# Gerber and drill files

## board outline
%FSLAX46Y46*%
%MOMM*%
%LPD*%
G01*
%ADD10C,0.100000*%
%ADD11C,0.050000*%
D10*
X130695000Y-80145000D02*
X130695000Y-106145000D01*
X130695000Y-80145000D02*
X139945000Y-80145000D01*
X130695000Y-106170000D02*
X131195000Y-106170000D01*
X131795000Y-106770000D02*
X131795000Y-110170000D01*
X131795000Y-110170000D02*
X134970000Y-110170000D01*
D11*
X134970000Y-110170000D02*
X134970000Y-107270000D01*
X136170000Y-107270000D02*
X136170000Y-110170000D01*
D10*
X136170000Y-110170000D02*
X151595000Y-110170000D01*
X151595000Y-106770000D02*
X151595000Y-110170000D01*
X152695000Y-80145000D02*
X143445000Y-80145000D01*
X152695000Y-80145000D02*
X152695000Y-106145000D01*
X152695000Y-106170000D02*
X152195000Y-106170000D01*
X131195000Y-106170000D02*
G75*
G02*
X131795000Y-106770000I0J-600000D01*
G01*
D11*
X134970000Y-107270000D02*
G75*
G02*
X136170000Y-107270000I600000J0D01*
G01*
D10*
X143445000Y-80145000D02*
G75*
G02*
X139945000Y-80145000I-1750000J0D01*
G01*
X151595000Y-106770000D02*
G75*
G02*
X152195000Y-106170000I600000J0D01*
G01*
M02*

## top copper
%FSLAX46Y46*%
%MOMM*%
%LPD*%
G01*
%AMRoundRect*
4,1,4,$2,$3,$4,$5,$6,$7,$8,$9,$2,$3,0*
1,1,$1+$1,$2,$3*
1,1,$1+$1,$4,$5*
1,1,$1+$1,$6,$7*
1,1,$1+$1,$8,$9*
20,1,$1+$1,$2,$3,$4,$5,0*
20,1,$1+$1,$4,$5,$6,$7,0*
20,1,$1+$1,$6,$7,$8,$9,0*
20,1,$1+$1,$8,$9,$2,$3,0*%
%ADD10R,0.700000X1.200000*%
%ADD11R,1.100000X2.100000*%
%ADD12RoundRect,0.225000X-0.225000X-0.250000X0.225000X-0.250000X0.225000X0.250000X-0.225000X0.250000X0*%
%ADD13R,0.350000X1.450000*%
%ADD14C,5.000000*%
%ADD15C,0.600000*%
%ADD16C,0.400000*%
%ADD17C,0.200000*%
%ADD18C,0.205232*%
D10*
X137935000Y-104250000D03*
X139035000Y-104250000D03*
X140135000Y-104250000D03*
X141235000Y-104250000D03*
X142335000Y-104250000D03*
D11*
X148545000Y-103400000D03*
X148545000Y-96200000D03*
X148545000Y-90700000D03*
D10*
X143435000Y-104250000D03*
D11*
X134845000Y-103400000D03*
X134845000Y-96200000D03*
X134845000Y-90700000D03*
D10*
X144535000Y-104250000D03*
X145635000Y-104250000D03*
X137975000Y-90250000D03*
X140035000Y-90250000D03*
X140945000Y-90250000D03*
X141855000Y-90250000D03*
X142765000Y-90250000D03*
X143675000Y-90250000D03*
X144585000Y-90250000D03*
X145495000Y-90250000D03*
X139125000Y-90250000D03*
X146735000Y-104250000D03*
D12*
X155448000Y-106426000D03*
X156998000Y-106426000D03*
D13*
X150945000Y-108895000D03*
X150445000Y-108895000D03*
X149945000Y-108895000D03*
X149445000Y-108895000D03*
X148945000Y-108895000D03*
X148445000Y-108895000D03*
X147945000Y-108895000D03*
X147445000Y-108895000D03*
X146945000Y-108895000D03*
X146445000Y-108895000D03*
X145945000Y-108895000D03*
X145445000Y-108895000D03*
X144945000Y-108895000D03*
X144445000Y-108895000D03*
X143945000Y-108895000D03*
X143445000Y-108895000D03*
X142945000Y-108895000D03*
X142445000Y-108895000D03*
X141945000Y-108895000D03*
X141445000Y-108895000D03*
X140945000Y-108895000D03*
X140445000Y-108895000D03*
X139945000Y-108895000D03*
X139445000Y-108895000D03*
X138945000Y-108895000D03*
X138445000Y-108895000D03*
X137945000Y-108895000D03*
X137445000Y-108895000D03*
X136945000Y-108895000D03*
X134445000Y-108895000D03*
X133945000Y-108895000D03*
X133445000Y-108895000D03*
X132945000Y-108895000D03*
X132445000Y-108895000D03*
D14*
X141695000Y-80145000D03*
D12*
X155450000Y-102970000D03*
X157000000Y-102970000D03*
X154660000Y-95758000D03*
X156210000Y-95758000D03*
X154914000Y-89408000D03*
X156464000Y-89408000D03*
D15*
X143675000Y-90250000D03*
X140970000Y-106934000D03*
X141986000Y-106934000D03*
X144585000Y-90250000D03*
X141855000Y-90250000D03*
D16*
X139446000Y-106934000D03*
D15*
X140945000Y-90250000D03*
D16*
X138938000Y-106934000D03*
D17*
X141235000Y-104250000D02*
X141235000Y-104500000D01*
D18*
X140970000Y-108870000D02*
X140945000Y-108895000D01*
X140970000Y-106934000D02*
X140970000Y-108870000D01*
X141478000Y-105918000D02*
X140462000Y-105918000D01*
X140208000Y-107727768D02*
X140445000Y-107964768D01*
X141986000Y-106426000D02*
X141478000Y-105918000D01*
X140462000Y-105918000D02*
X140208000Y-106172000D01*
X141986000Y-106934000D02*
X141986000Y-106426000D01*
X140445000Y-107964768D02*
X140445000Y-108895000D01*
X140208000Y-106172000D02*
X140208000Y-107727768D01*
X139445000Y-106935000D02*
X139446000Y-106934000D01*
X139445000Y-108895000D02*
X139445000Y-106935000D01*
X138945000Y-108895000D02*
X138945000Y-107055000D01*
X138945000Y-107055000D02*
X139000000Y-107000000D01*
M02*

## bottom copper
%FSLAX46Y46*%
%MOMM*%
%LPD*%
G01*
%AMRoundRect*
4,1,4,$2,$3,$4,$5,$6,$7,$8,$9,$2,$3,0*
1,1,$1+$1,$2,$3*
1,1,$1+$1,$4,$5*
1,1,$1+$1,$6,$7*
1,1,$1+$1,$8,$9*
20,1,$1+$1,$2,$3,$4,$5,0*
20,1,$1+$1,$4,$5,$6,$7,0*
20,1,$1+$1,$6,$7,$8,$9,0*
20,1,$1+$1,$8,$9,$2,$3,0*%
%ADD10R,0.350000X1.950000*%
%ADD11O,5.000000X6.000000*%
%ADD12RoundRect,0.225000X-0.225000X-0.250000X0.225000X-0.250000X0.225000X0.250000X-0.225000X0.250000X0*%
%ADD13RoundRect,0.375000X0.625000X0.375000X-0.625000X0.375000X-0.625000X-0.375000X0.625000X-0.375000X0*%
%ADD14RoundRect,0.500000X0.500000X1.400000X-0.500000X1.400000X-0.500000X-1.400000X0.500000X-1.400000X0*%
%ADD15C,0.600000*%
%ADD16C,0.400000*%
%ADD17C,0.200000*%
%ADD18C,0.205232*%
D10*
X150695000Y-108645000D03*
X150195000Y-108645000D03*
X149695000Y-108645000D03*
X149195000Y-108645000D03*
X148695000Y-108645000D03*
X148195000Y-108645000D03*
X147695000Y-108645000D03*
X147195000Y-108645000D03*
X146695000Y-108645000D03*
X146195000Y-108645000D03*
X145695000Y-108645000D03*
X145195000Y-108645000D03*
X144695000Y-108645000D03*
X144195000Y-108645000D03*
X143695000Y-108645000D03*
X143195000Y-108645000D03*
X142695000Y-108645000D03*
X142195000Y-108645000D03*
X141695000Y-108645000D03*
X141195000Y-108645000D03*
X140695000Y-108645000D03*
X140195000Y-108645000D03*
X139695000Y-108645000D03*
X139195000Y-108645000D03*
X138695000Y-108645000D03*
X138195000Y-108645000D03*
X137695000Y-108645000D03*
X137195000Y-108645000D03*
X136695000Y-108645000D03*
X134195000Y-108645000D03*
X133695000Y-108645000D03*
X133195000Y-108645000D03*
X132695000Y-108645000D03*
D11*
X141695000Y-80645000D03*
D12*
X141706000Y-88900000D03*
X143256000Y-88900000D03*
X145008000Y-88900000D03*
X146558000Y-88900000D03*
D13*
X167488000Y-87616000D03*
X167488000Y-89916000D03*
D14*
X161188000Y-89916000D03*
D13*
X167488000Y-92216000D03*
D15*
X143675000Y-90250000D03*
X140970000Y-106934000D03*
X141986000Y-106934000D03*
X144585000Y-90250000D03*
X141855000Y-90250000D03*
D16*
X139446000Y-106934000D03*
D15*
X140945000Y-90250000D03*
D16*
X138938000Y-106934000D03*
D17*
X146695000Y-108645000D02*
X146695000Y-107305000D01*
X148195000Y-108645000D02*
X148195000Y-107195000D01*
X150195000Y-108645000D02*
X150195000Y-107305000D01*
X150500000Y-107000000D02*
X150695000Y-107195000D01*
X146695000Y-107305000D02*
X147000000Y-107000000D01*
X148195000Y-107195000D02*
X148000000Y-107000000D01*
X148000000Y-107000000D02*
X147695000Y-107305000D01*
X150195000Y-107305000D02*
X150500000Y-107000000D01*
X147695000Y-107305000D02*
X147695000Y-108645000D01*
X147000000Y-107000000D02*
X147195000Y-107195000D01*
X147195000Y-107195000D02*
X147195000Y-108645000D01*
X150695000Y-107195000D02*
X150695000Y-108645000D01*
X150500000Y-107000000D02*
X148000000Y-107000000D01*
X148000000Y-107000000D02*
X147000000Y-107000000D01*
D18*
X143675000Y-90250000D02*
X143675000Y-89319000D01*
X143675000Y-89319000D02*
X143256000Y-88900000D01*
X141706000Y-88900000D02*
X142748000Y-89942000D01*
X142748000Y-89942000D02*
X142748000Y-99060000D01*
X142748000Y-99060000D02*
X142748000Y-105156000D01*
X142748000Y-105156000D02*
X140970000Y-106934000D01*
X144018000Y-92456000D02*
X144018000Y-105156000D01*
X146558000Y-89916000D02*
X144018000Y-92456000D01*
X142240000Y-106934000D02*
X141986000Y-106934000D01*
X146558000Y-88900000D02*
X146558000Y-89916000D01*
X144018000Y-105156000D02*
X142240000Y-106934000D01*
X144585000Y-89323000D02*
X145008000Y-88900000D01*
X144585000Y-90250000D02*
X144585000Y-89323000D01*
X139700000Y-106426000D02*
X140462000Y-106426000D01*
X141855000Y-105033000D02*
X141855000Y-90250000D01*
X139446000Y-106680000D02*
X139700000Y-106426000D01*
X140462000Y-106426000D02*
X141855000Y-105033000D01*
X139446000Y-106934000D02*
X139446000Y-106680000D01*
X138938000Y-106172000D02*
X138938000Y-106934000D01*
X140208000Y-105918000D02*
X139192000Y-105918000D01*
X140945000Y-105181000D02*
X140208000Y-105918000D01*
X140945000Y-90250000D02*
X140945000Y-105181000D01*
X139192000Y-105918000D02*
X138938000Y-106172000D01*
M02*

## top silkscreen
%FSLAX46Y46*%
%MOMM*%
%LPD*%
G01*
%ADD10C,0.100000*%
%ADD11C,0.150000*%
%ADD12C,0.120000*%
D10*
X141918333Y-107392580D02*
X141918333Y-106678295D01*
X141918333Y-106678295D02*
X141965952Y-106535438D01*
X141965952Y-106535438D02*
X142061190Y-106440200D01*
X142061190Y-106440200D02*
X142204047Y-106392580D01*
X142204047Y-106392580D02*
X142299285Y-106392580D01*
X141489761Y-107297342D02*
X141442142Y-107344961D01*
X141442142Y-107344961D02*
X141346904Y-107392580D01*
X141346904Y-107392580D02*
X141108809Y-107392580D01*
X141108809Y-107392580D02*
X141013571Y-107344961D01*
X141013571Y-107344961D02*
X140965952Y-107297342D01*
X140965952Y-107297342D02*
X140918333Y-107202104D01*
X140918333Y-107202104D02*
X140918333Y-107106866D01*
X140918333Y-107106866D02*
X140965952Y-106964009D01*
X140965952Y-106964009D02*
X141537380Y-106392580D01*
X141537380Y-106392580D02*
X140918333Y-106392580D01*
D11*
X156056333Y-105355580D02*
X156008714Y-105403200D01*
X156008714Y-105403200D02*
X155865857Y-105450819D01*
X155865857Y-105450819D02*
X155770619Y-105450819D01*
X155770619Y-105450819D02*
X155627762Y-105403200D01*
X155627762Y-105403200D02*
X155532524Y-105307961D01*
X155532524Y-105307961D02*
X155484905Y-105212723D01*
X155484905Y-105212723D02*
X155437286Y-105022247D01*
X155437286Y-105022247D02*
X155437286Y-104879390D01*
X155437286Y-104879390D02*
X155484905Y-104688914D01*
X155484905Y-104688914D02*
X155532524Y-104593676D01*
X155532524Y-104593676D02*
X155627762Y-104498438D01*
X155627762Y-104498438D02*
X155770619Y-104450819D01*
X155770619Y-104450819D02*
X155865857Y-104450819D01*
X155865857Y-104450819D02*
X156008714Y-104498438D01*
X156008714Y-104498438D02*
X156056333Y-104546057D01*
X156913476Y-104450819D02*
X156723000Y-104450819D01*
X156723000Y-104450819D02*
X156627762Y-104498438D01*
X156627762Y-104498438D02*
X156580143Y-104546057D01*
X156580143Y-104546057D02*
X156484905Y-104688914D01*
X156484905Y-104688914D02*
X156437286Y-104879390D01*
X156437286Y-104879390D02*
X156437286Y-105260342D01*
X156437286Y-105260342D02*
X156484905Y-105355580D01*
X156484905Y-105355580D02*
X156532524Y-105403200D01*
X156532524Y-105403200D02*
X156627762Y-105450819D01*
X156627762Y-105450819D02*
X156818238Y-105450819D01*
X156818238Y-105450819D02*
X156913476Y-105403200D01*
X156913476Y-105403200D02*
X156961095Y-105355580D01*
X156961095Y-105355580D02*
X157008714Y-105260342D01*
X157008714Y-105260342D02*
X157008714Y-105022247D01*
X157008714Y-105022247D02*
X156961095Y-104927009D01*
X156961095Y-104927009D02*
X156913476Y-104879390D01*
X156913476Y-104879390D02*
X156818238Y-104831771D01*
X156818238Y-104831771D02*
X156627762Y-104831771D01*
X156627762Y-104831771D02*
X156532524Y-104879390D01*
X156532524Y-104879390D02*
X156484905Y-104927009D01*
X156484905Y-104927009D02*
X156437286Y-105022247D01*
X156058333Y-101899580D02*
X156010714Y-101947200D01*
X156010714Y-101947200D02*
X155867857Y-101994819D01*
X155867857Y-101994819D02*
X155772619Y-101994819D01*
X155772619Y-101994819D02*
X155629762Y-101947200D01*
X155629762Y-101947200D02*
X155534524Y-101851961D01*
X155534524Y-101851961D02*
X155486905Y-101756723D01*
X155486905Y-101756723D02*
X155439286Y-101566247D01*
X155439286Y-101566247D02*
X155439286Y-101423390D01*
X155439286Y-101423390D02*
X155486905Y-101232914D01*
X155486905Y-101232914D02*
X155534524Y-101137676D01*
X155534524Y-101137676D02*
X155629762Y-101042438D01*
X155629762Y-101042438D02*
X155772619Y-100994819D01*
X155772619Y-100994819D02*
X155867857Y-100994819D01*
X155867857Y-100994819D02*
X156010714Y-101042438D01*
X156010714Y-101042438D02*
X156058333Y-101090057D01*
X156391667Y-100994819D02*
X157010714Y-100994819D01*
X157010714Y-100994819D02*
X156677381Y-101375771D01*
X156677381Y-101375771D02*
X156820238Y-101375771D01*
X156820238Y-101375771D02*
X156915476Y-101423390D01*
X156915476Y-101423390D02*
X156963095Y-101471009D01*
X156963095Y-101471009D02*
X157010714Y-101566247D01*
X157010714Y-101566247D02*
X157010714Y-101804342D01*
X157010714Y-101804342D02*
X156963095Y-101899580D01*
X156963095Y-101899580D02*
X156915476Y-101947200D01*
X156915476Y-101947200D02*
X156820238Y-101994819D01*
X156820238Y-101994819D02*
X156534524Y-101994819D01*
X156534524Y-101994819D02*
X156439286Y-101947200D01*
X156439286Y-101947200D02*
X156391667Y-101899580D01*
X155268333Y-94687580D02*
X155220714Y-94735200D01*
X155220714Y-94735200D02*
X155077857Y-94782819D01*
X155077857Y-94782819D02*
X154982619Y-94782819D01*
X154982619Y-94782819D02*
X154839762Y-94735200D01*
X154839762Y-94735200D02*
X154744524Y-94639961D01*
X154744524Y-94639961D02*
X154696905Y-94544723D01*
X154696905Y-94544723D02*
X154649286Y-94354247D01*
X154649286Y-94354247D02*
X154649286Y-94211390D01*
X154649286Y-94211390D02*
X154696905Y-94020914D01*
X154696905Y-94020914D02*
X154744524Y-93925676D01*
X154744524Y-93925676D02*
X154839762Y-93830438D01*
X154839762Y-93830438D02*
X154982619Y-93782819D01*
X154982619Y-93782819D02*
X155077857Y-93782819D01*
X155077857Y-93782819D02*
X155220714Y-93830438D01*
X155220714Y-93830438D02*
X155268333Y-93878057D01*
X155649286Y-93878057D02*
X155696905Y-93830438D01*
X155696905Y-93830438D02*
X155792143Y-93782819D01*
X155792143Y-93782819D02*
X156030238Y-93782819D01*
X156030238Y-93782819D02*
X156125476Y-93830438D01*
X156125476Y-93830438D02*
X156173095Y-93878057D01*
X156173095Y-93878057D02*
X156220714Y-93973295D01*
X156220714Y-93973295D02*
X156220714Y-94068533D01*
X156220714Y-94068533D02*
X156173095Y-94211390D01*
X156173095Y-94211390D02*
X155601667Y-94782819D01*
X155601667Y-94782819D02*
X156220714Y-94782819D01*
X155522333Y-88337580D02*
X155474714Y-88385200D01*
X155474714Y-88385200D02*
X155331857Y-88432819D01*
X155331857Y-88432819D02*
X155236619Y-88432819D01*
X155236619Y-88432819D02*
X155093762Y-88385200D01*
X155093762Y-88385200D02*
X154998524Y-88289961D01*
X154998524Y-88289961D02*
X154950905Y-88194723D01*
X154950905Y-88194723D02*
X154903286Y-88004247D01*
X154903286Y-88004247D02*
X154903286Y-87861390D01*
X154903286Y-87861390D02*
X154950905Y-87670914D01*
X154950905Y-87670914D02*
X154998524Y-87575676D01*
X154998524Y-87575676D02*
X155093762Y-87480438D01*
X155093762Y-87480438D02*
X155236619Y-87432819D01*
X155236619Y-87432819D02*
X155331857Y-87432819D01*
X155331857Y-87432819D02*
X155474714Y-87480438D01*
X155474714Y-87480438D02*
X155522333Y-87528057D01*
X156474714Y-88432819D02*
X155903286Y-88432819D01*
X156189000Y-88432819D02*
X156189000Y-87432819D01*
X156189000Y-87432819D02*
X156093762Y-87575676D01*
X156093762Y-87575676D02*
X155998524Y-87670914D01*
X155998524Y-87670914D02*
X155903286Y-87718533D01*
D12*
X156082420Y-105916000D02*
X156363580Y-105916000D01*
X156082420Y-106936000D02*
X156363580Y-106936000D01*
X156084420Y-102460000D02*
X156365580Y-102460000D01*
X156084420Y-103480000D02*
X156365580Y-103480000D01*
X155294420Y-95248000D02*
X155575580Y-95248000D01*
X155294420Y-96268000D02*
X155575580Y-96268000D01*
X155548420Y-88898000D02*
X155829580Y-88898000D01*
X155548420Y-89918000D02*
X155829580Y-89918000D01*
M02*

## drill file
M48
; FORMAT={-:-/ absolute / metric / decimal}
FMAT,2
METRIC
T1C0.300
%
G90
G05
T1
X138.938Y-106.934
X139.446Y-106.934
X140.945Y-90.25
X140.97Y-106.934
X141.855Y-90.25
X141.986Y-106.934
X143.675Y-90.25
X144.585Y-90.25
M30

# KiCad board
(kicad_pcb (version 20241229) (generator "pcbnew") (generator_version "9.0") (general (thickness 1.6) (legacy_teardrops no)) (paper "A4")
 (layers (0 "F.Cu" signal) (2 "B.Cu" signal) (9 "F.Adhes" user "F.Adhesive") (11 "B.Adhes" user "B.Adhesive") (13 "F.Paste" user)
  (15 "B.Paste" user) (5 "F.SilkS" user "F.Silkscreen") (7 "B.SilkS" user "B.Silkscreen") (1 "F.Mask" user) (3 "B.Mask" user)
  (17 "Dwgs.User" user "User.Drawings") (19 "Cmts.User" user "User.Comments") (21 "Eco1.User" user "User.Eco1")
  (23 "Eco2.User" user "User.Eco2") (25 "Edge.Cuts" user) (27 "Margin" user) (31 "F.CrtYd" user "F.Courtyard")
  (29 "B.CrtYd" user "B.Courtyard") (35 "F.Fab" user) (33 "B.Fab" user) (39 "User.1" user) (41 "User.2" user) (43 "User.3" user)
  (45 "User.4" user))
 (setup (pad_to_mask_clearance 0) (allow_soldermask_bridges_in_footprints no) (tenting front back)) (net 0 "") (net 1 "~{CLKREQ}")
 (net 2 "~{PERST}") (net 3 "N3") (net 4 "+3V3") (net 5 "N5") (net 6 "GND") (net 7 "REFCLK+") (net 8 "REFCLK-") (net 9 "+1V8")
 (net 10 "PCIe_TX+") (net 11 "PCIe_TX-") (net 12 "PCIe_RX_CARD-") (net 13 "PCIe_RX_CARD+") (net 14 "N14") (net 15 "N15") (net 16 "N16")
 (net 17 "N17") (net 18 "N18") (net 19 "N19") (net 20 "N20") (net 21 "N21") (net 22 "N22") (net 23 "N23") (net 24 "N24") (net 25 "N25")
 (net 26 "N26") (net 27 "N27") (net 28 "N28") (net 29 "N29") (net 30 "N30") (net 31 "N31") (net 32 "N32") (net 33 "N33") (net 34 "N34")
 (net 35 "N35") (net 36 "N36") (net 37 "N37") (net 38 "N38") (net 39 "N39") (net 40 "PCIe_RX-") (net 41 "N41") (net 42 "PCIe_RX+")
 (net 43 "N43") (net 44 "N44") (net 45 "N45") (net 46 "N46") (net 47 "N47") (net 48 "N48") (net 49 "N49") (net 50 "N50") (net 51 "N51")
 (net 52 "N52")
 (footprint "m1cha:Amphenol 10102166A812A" (layer "F.Cu") (at 141.695 104.25 180)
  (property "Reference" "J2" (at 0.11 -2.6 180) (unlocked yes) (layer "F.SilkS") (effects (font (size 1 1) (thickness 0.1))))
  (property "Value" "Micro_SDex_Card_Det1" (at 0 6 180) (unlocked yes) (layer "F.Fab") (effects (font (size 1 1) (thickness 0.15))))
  (pad "1" smd rect (at 3.76 0 180) (size 0.7 1.2) (layers "F.Cu" "F.Mask" "F.Paste") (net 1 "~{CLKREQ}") (thermal_bridge_angle 45))
  (pad "2" smd rect (at 2.66 0 180) (size 0.7 1.2) (layers "F.Cu" "F.Mask" "F.Paste") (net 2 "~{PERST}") (thermal_bridge_angle 45))
  (pad "3" smd rect (at 1.56 0 180) (size 0.7 1.2) (layers "F.Cu" "F.Mask" "F.Paste") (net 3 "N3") (thermal_bridge_angle 45))
  (pad "4" smd rect (at 0.46 0 180) (size 0.7 1.2) (layers "F.Cu" "F.Mask" "F.Paste") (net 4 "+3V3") (thermal_bridge_angle 45))
  (pad "5" smd rect (at -0.64 0 180) (size 0.7 1.2) (layers "F.Cu" "F.Mask" "F.Paste") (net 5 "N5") (thermal_bridge_angle 45))
  (pad "6" smd rect (at -6.85 0.85 180) (size 1.1 2.1) (layers "F.Cu" "F.Mask" "F.Paste") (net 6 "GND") (thermal_bridge_angle 45))
  (pad "6" smd rect (at -6.85 8.05 180) (size 1.1 2.1) (layers "F.Cu" "F.Mask" "F.Paste") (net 6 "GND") (thermal_bridge_angle 45))
  (pad "6" smd rect (at -6.85 13.55 180) (size 1.1 2.1) (layers "F.Cu" "F.Mask" "F.Paste") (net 6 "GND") (thermal_bridge_angle 45))
  (pad "6" smd rect (at -1.74 0 180) (size 0.7 1.2) (layers "F.Cu" "F.Mask" "F.Paste") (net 6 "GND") (thermal_bridge_angle 45))
  (pad "6" smd rect (at 6.85 0.85 180) (size 1.1 2.1) (layers "F.Cu" "F.Mask" "F.Paste") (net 6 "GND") (thermal_bridge_angle 45))
  (pad "6" smd rect (at 6.85 8.05 180) (size 1.1 2.1) (layers "F.Cu" "F.Mask" "F.Paste") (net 6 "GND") (thermal_bridge_angle 45))
  (pad "6" smd rect (at 6.85 13.55 180) (size 1.1 2.1) (layers "F.Cu" "F.Mask" "F.Paste") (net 6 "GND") (thermal_bridge_angle 45))
  (pad "7" smd rect (at -2.84 0 180) (size 0.7 1.2) (layers "F.Cu" "F.Mask" "F.Paste") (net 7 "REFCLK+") (thermal_bridge_angle 45))
  (pad "8" smd rect (at -3.94 0 180) (size 0.7 1.2) (layers "F.Cu" "F.Mask" "F.Paste") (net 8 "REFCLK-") (thermal_bridge_angle 45))
  (pad "9" smd rect (at 3.72 14 180) (size 0.7 1.2) (layers "F.Cu" "F.Mask" "F.Paste") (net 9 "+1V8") (thermal_bridge_angle 45))
  (pad "10" smd rect (at 1.66 14 180) (size 0.7 1.2) (layers "F.Cu" "F.Mask" "F.Paste") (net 6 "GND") (thermal_bridge_angle 45))
  (pad "11" smd rect (at 0.75 14 180) (size 0.7 1.2) (layers "F.Cu" "F.Mask" "F.Paste") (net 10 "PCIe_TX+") (thermal_bridge_angle 45))
  (pad "12" smd rect (at -0.16 14 180) (size 0.7 1.2) (layers "F.Cu" "F.Mask" "F.Paste") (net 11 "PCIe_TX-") (thermal_bridge_angle 45))
  (pad "13" smd rect (at -1.07 14 180) (size 0.7 1.2) (layers "F.Cu" "F.Mask" "F.Paste") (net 6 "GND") (thermal_bridge_angle 45))
  (pad "14" smd rect (at -1.98 14 180) (size 0.7 1.2) (layers "F.Cu" "F.Mask" "F.Paste") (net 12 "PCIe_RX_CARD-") (thermal_bridge_angle 45))
  (pad "15" smd rect (at -2.89 14 180) (size 0.7 1.2) (layers "F.Cu" "F.Mask" "F.Paste") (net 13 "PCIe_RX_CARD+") (thermal_bridge_angle 45))
  (pad "16" smd rect (at -3.8 14 180) (size 0.7 1.2) (layers "F.Cu" "F.Mask" "F.Paste") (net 6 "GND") (thermal_bridge_angle 45))
  (pad "17" smd rect (at 2.57 14 180) (size 0.7 1.2) (layers "F.Cu" "F.Mask" "F.Paste") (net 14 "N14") (thermal_bridge_angle 45))
  (pad "18" smd rect (at -5.04 0 180) (size 0.7 1.2) (layers "F.Cu" "F.Mask" "F.Paste") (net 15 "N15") (thermal_bridge_angle 45))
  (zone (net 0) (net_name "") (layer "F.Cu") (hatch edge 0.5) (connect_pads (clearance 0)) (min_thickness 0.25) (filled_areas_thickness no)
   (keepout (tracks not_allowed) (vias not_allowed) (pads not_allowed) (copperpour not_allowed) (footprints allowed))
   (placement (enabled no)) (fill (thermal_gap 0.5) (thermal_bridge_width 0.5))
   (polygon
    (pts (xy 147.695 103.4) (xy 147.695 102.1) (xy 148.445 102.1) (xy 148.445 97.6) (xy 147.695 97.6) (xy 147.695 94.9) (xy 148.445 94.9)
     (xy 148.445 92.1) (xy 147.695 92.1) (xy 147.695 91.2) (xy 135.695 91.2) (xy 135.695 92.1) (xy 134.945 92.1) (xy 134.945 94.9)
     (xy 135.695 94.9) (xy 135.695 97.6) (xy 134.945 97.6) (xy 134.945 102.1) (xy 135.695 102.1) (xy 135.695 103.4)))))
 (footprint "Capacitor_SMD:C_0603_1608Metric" (layer "F.Cu") (at 156.223 106.426)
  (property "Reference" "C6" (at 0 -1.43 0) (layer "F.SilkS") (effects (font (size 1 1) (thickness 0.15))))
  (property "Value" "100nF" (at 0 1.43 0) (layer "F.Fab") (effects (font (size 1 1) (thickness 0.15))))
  (fp_line (start -0.14058 -0.51) (end 0.14058 -0.51) (stroke (width 0.12) (type solid)) (layer "F.SilkS"))
  (fp_line (start -0.14058 0.51) (end 0.14058 0.51) (stroke (width 0.12) (type solid)) (layer "F.SilkS"))
  (pad "1" smd roundrect (at -0.775 0) (size 0.9 0.95) (layers "F.Cu" "F.Mask" "F.Paste") (roundrect_rratio 0.25) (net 9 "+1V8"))
  (pad "2" smd roundrect (at 0.775 0) (size 0.9 0.95) (layers "F.Cu" "F.Mask" "F.Paste") (roundrect_rratio 0.25) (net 6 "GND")))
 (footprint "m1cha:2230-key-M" (layer "F.Cu") (at 141.695 79.145)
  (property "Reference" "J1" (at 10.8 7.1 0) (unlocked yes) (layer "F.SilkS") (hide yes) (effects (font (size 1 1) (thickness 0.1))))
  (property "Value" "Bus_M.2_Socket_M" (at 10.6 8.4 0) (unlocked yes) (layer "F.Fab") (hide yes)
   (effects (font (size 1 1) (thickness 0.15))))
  (fp_line (start -11 1) (end -11 27) (stroke (width 0.1) (type solid)) (layer "Edge.Cuts"))
  (fp_line (start -11 1) (end -1.75 1) (stroke (width 0.1) (type default)) (layer "Edge.Cuts"))
  (fp_line (start -11 27.025) (end -10.5 27.025) (stroke (width 0.1) (type default)) (layer "Edge.Cuts"))
  (fp_line (start -9.9 27.625) (end -9.9 31.025) (stroke (width 0.1) (type default)) (layer "Edge.Cuts"))
  (fp_line (start -9.9 31.025) (end -6.725 31.025) (stroke (width 0.1) (type solid)) (layer "Edge.Cuts"))
  (fp_line (start -6.725 31.025) (end -6.725 28.125) (stroke (width 0.05) (type default)) (layer "Edge.Cuts"))
  (fp_line (start -5.525 28.125) (end -5.525 31.025) (stroke (width 0.05) (type default)) (layer "Edge.Cuts"))
  (fp_line (start -5.525 31.025) (end 9.9 31.025) (stroke (width 0.1) (type solid)) (layer "Edge.Cuts"))
  (fp_line (start 9.9 27.625) (end 9.9 31.025) (stroke (width 0.1) (type default)) (layer "Edge.Cuts"))
  (fp_line (start 11 1) (end 1.75 1) (stroke (width 0.1) (type default)) (layer "Edge.Cuts"))
  (fp_line (start 11 1) (end 11 27) (stroke (width 0.1) (type solid)) (layer "Edge.Cuts"))
  (fp_line (start 11 27.025) (end 10.5 27.025) (stroke (width 0.1) (type default)) (layer "Edge.Cuts"))
  (fp_arc (start -10.5 27.025) (mid -10.075736 27.200736) (end -9.9 27.625) (stroke (width 0.1) (type default)) (layer "Edge.Cuts"))
  (fp_arc (start -6.725 28.125) (mid -6.125 27.525) (end -5.525 28.125) (stroke (width 0.05) (type default)) (layer "Edge.Cuts"))
  (fp_arc (start 1.75 1) (mid 0 2.75) (end -1.75 1) (stroke (width 0.1) (type default)) (layer "Edge.Cuts"))
  (fp_arc (start 9.9 27.625) (mid 10.075736 27.200736) (end 10.5 27.025) (stroke (width 0.1) (type default)) (layer "Edge.Cuts"))
  (pad "1" connect rect (at 9.25 29.75) (size 0.35 1.45) (layers "F.Cu" "F.Mask") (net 6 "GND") (thermal_bridge_angle 45))
  (pad "2" connect rect (at 9 29.5) (size 0.35 1.95) (layers "B.Cu" "B.Mask") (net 4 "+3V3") (thermal_bridge_angle 45))
  (pad "3" connect rect (at 8.75 29.75) (size 0.35 1.45) (layers "F.Cu" "F.Mask") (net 6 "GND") (thermal_bridge_angle 45))
  (pad "4" connect rect (at 8.5 29.5) (size 0.35 1.95) (layers "B.Cu" "B.Mask") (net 4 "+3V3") (thermal_bridge_angle 45))
  (pad "5" connect rect (at 8.25 29.75) (size 0.35 1.45) (layers "F.Cu" "F.Mask") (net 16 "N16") (thermal_bridge_angle 45))
  (pad "6" connect rect (at 8 29.5) (size 0.35 1.95) (layers "B.Cu" "B.Mask") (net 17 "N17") (thermal_bridge_angle 45))
  (pad "7" connect rect (at 7.75 29.75) (size 0.35 1.45) (layers "F.Cu" "F.Mask") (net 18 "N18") (thermal_bridge_angle 45))
  (pad "8" connect rect (at 7.5 29.5) (size 0.35 1.95) (layers "B.Cu" "B.Mask") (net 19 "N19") (thermal_bridge_angle 45))
  (pad "9" connect rect (at 7.25 29.75) (size 0.35 1.45) (layers "F.Cu" "F.Mask") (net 6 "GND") (thermal_bridge_angle 45))
  (pad "10" connect rect (at 7 29.5) (size 0.35 1.95) (layers "B.Cu" "B.Mask") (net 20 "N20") (thermal_bridge_angle 45))
  (pad "11" connect rect (at 6.75 29.75) (size 0.35 1.45) (layers "F.Cu" "F.Mask") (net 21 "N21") (thermal_bridge_angle 45))
  (pad "12" connect rect (at 6.5 29.5) (size 0.35 1.95) (layers "B.Cu" "B.Mask") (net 4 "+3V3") (thermal_bridge_angle 45))
  (pad "13" connect rect (at 6.25 29.75) (size 0.35 1.45) (layers "F.Cu" "F.Mask") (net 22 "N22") (thermal_bridge_angle 45))
  (pad "14" connect rect (at 6 29.5) (size 0.35 1.95) (layers "B.Cu" "B.Mask") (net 4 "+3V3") (thermal_bridge_angle 45))
  (pad "15" connect rect (at 5.75 29.75) (size 0.35 1.45) (layers "F.Cu" "F.Mask") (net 6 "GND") (thermal_bridge_angle 45))
  (pad "16" connect rect (at 5.5 29.5) (size 0.35 1.95) (layers "B.Cu" "B.Mask") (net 4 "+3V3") (thermal_bridge_angle 45))
  (pad "17" connect rect (at 5.25 29.75) (size 0.35 1.45) (layers "F.Cu" "F.Mask") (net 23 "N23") (thermal_bridge_angle 45))
  (pad "18" connect rect (at 5 29.5) (size 0.35 1.95) (layers "B.Cu" "B.Mask") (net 4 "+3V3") (thermal_bridge_angle 45))
  (pad "19" connect rect (at 4.75 29.75) (size 0.35 1.45) (layers "F.Cu" "F.Mask") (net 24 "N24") (thermal_bridge_angle 45))
  (pad "20" connect rect (at 4.5 29.5) (size 0.35 1.95) (layers "B.Cu" "B.Mask") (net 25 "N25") (thermal_bridge_angle 45))
  (pad "21" connect rect (at 4.25 29.75) (size 0.35 1.45) (layers "F.Cu" "F.Mask") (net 6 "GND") (thermal_bridge_angle 45))
  (pad "22" connect rect (at 4 29.5) (size 0.35 1.95) (layers "B.Cu" "B.Mask") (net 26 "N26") (thermal_bridge_angle 45))
  (pad "23" connect rect (at 3.75 29.75) (size 0.35 1.45) (layers "F.Cu" "F.Mask") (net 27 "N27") (thermal_bridge_angle 45))
  (pad "24" connect rect (at 3.5 29.5) (size 0.35 1.95) (layers "B.Cu" "B.Mask") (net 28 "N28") (thermal_bridge_angle 45))
  (pad "25" connect rect (at 3.25 29.75) (size 0.35 1.45) (layers "F.Cu" "F.Mask") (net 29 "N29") (thermal_bridge_angle 45))
  (pad "26" connect rect (at 3 29.5) (size 0.35 1.95) (layers "B.Cu" "B.Mask") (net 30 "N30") (thermal_bridge_angle 45))
  (pad "27" connect rect (at 2.75 29.75) (size 0.35 1.45) (layers "F.Cu" "F.Mask") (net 6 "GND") (thermal_bridge_angle 45))
  (pad "28" connect rect (at 2.5 29.5) (size 0.35 1.95) (layers "B.Cu" "B.Mask") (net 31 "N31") (thermal_bridge_angle 45))
  (pad "29" connect rect (at 2.25 29.75) (size 0.35 1.45) (layers "F.Cu" "F.Mask") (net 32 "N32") (thermal_bridge_angle 45))
  (pad "30" connect rect (at 2 29.5) (size 0.35 1.95) (layers "B.Cu" "B.Mask") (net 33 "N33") (thermal_bridge_angle 45))
  (pad "31" connect rect (at 1.75 29.75) (size 0.35 1.45) (layers "F.Cu" "F.Mask") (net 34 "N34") (thermal_bridge_angle 45))
  (pad "32" connect rect (at 1.5 29.5) (size 0.35 1.95) (layers "B.Cu" "B.Mask") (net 6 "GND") (thermal_bridge_angle 45))
  (pad "33" connect rect (at 1.25 29.75) (size 0.35 1.45) (layers "F.Cu" "F.Mask") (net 6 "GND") (thermal_bridge_angle 45))
  (pad "34" connect rect (at 1 29.5) (size 0.35 1.95) (layers "B.Cu" "B.Mask") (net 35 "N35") (thermal_bridge_angle 45))
  (pad "35" connect rect (at 0.75 29.75) (size 0.35 1.45) (layers "F.Cu" "F.Mask") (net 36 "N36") (thermal_bridge_angle 45))
  (pad "36" connect rect (at 0.5 29.5) (size 0.35 1.95) (layers "B.Cu" "B.Mask") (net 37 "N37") (thermal_bridge_angle 45))
  (pad "37" connect rect (at 0.25 29.75) (size 0.35 1.45) (layers "F.Cu" "F.Mask") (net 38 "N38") (thermal_bridge_angle 45))
  (pad "38" connect rect (at 0 29.5) (size 0.35 1.95) (layers "B.Cu" "B.Mask") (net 6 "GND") (thermal_bridge_angle 45))
  (pad "39" connect rect (at -0.25 29.75) (size 0.35 1.45) (layers "F.Cu" "F.Mask") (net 6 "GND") (thermal_bridge_angle 45))
  (pad "40" connect rect (at -0.5 29.5) (size 0.35 1.95) (layers "B.Cu" "B.Mask") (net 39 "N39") (thermal_bridge_angle 45))
  (pad "41" connect rect (at -0.75 29.75) (size 0.35 1.45) (layers "F.Cu" "F.Mask") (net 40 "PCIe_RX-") (thermal_bridge_angle 45))
  (pad "42" connect rect (at -1 29.5) (size 0.35 1.95) (layers "B.Cu" "B.Mask") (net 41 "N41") (thermal_bridge_angle 45))
  (pad "43" connect rect (at -1.25 29.75) (size 0.35 1.45) (layers "F.Cu" "F.Mask") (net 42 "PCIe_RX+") (thermal_bridge_angle 45))
  (pad "44" connect rect (at -1.5 29.5) (size 0.35 1.95) (layers "B.Cu" "B.Mask") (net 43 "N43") (thermal_bridge_angle 45))
  (pad "45" connect rect (at -1.75 29.75) (size 0.35 1.45) (layers "F.Cu" "F.Mask") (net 6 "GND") (thermal_bridge_angle 45))
  (pad "46" connect rect (at -2 29.5) (size 0.35 1.95) (layers "B.Cu" "B.Mask") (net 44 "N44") (thermal_bridge_angle 45))
  (pad "47" connect rect (at -2.25 29.75) (size 0.35 1.45) (layers "F.Cu" "F.Mask") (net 11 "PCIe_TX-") (thermal_bridge_angle 45))
  (pad "48" connect rect (at -2.5 29.5) (size 0.35 1.95) (layers "B.Cu" "B.Mask") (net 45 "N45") (thermal_bridge_angle 45))
  (pad "49" connect rect (at -2.75 29.75) (size 0.35 1.45) (layers "F.Cu" "F.Mask") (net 10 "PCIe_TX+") (thermal_bridge_angle 45))
  (pad "50" connect rect (at -3 29.5) (size 0.35 1.95) (layers "B.Cu" "B.Mask") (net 2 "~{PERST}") (thermal_bridge_angle 45))
  (pad "51" connect rect (at -3.25 29.75) (size 0.35 1.45) (layers "F.Cu" "F.Mask") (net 6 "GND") (thermal_bridge_angle 45))
  (pad "52" connect rect (at -3.5 29.5) (size 0.35 1.95) (layers "B.Cu" "B.Mask") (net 1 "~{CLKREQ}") (thermal_bridge_angle 45))
  (pad "53" connect rect (at -3.75 29.75) (size 0.35 1.45) (layers "F.Cu" "F.Mask") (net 8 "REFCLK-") (thermal_bridge_angle 45))
  (pad "54" connect rect (at -4 29.5) (size 0.35 1.95) (layers "B.Cu" "B.Mask") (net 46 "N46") (thermal_bridge_angle 45))
  (pad "55" connect rect (at -4.25 29.75) (size 0.35 1.45) (layers "F.Cu" "F.Mask") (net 7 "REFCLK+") (thermal_bridge_angle 45))
  (pad "56" connect rect (at -4.5 29.5) (size 0.35 1.95) (layers "B.Cu" "B.Mask") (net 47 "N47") (thermal_bridge_angle 45))
  (pad "57" connect rect (at -4.75 29.75) (size 0.35 1.45) (layers "F.Cu" "F.Mask") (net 6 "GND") (thermal_bridge_angle 45))
  (pad "58" connect rect (at -5 29.5) (size 0.35 1.95) (layers "B.Cu" "B.Mask") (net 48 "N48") (thermal_bridge_angle 45))
  (pad "67" connect rect (at -7.25 29.75) (size 0.35 1.45) (layers "F.Cu" "F.Mask") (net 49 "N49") (thermal_bridge_angle 45))
  (pad "68" connect rect (at -7.5 29.5) (size 0.35 1.95) (layers "B.Cu" "B.Mask") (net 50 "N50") (thermal_bridge_angle 45))
  (pad "69" connect rect (at -7.75 29.75) (size 0.35 1.45) (layers "F.Cu" "F.Mask") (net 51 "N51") (thermal_bridge_angle 45))
  (pad "70" connect rect (at -8 29.5) (size 0.35 1.95) (layers "B.Cu" "B.Mask") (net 4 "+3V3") (thermal_bridge_angle 45))
  (pad "71" connect rect (at -8.25 29.75) (size 0.35 1.45) (layers "F.Cu" "F.Mask") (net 6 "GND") (thermal_bridge_angle 45))
  (pad "72" connect rect (at -8.5 29.5) (size 0.35 1.95) (layers "B.Cu" "B.Mask") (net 4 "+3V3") (thermal_bridge_angle 45))
  (pad "73" connect rect (at -8.75 29.75) (size 0.35 1.45) (layers "F.Cu" "F.Mask") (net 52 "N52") (thermal_bridge_angle 45))
  (pad "74" connect rect (at -9 29.5) (size 0.35 1.95) (layers "B.Cu" "B.Mask") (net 4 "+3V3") (thermal_bridge_angle 45))
  (pad "75" connect rect (at -9.25 29.75) (size 0.35 1.45) (layers "F.Cu" "F.Mask") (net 6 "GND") (thermal_bridge_angle 45))
  (pad "76" connect circle (at 0 1) (size 5 5) (layers "F.Cu" "F.Mask") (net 6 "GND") (zone_connect 2))
  (pad "77" connect oval (at 0 1.5) (size 5 6) (layers "B.Cu" "B.Mask") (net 6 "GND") (zone_connect 2)))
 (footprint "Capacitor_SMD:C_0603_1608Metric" (layer "F.Cu") (at 156.225 102.97)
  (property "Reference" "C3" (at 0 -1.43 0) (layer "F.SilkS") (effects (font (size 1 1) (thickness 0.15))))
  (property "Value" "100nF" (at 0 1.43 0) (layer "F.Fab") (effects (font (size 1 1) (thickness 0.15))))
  (fp_line (start -0.14058 -0.51) (end 0.14058 -0.51) (stroke (width 0.12) (type solid)) (layer "F.SilkS"))
  (fp_line (start -0.14058 0.51) (end 0.14058 0.51) (stroke (width 0.12) (type solid)) (layer "F.SilkS"))
  (pad "1" smd roundrect (at -0.775 0) (size 0.9 0.95) (layers "F.Cu" "F.Mask" "F.Paste") (roundrect_rratio 0.25) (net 4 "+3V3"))
  (pad "2" smd roundrect (at 0.775 0) (size 0.9 0.95) (layers "F.Cu" "F.Mask" "F.Paste") (roundrect_rratio 0.25) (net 6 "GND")))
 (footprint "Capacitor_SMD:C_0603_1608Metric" (layer "F.Cu") (at 155.435 95.758)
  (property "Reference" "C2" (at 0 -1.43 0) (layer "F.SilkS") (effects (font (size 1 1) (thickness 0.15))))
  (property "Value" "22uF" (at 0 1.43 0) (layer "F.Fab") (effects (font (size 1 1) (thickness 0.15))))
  (fp_line (start -0.14058 -0.51) (end 0.14058 -0.51) (stroke (width 0.12) (type solid)) (layer "F.SilkS"))
  (fp_line (start -0.14058 0.51) (end 0.14058 0.51) (stroke (width 0.12) (type solid)) (layer "F.SilkS"))
  (pad "1" smd roundrect (at -0.775 0) (size 0.9 0.95) (layers "F.Cu" "F.Mask" "F.Paste") (roundrect_rratio 0.25) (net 9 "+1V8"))
  (pad "2" smd roundrect (at 0.775 0) (size 0.9 0.95) (layers "F.Cu" "F.Mask" "F.Paste") (roundrect_rratio 0.25) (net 6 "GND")))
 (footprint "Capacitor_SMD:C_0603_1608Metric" (layer "F.Cu") (at 155.689 89.408)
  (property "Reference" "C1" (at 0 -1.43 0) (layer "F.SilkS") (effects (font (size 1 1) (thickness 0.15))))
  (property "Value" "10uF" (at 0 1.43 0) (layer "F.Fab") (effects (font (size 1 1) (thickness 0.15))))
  (fp_line (start -0.14058 -0.51) (end 0.14058 -0.51) (stroke (width 0.12) (type solid)) (layer "F.SilkS"))
  (fp_line (start -0.14058 0.51) (end 0.14058 0.51) (stroke (width 0.12) (type solid)) (layer "F.SilkS"))
  (pad "1" smd roundrect (at -0.775 0) (size 0.9 0.95) (layers "F.Cu" "F.Mask" "F.Paste") (roundrect_rratio 0.25) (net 4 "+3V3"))
  (pad "2" smd roundrect (at 0.775 0) (size 0.9 0.95) (layers "F.Cu" "F.Mask" "F.Paste") (roundrect_rratio 0.25) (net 6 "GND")))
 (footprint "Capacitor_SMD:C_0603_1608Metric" (layer "B.Cu") (at 142.481 88.9)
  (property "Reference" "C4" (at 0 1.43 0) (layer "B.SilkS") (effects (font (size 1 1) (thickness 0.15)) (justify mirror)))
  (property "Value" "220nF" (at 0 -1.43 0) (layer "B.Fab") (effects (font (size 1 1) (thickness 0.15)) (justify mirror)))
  (pad "1" smd roundrect (at -0.775 0) (size 0.9 0.95) (layers "B.Cu" "B.Mask" "B.Paste") (roundrect_rratio 0.25) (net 40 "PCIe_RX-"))
  (pad "2" smd roundrect (at 0.775 0) (size 0.9 0.95) (layers "B.Cu" "B.Mask" "B.Paste") (roundrect_rratio 0.25) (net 12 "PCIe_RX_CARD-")))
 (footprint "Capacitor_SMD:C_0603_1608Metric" (layer "B.Cu") (at 145.783 88.9)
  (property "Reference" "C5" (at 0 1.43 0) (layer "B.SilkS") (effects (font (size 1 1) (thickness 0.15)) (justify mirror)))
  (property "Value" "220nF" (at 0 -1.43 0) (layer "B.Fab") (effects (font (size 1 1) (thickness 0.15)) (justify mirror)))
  (pad "1" smd roundrect (at -0.775 0) (size 0.9 0.95) (layers "B.Cu" "B.Mask" "B.Paste") (roundrect_rratio 0.25) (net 13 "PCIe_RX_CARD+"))
  (pad "2" smd roundrect (at 0.775 0) (size 0.9 0.95) (layers "B.Cu" "B.Mask" "B.Paste") (roundrect_rratio 0.25) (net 42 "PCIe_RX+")))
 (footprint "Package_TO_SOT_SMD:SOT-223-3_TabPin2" (layer "B.Cu") (at 164.338 89.916 180)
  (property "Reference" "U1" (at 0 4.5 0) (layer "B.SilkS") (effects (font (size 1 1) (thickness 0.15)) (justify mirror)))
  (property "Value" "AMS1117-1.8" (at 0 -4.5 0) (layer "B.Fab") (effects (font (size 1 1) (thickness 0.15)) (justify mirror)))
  (pad "1" smd roundrect (at -3.15 2.3 180) (size 2 1.5) (layers "B.Cu" "B.Mask" "B.Paste") (roundrect_rratio 0.25) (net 6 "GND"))
  (pad "2" smd roundrect (at -3.15 0 180) (size 2 1.5) (layers "B.Cu" "B.Mask" "B.Paste") (roundrect_rratio 0.25) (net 9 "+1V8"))
  (pad "2" smd roundrect (at 3.15 0 180) (size 2 3.8) (layers "B.Cu" "B.Mask" "B.Paste") (roundrect_rratio 0.25) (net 9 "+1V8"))
  (pad "3" smd roundrect (at -3.15 -2.3 180) (size 2 1.5) (layers "B.Cu" "B.Mask" "B.Paste") (roundrect_rratio 0.25) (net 4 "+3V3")))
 (segment (start 141.235 104.25) (end 141.235 104.5) (width 0.2) (layer "F.Cu") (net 4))
 (segment (start 146.695 108.645) (end 146.695 107.305) (width 0.2) (layer "B.Cu") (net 4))
 (segment (start 148.195 108.645) (end 148.195 107.195) (width 0.2) (layer "B.Cu") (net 4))
 (segment (start 150.195 108.645) (end 150.195 107.305) (width 0.2) (layer "B.Cu") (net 4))
 (segment (start 150.5 107) (end 150.695 107.195) (width 0.2) (layer "B.Cu") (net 4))
 (segment (start 146.695 107.305) (end 147 107) (width 0.2) (layer "B.Cu") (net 4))
 (segment (start 148.195 107.195) (end 148 107) (width 0.2) (layer "B.Cu") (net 4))
 (segment (start 148 107) (end 147.695 107.305) (width 0.2) (layer "B.Cu") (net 4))
 (segment (start 150.195 107.305) (end 150.5 107) (width 0.2) (layer "B.Cu") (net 4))
 (segment (start 147.695 107.305) (end 147.695 108.645) (width 0.2) (layer "B.Cu") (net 4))
 (segment (start 147 107) (end 147.195 107.195) (width 0.2) (layer "B.Cu") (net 4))
 (segment (start 147.195 107.195) (end 147.195 108.645) (width 0.2) (layer "B.Cu") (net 4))
 (segment (start 150.695 107.195) (end 150.695 108.645) (width 0.2) (layer "B.Cu") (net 4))
 (segment (start 150.5 107) (end 148 107) (width 0.2) (layer "B.Cu") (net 4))
 (segment (start 148 107) (end 147 107) (width 0.2) (layer "B.Cu") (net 4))
 (via (at 143.675 90.25) (size 0.6) (drill 0.3) (layers "F.Cu" "B.Cu") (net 12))
 (segment (start 143.675 90.25) (end 143.675 89.319) (width 0.205232) (layer "B.Cu") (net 12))
 (segment (start 143.675 89.319) (end 143.256 88.9) (width 0.205232) (layer "B.Cu") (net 12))
 (segment (start 140.97 108.87) (end 140.945 108.895) (width 0.205232) (layer "F.Cu") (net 40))
 (segment (start 140.97 106.934) (end 140.97 108.87) (width 0.205232) (layer "F.Cu") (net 40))
 (via (at 140.97 106.934) (size 0.6) (drill 0.3) (layers "F.Cu" "B.Cu") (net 40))
 (segment (start 141.706 88.9) (end 142.748 89.942) (width 0.205232) (layer "B.Cu") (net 40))
 (segment (start 142.748 89.942) (end 142.748 99.06) (width 0.205232) (layer "B.Cu") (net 40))
 (segment (start 142.748 99.06) (end 142.748 105.156) (width 0.205232) (layer "B.Cu") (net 40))
 (segment (start 142.748 105.156) (end 140.97 106.934) (width 0.205232) (layer "B.Cu") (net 40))
 (segment (start 141.478 105.918) (end 140.462 105.918) (width 0.205232) (layer "F.Cu") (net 42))
 (segment (start 140.208 107.727768) (end 140.445 107.964768) (width 0.205232) (layer "F.Cu") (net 42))
 (segment (start 141.986 106.426) (end 141.478 105.918) (width 0.205232) (layer "F.Cu") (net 42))
 (segment (start 140.462 105.918) (end 140.208 106.172) (width 0.205232) (layer "F.Cu") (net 42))
 (segment (start 141.986 106.934) (end 141.986 106.426) (width 0.205232) (layer "F.Cu") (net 42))
 (segment (start 140.445 107.964768) (end 140.445 108.895) (width 0.205232) (layer "F.Cu") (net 42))
 (segment (start 140.208 106.172) (end 140.208 107.727768) (width 0.205232) (layer "F.Cu") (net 42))
 (via (at 141.986 106.934) (size 0.6) (drill 0.3) (layers "F.Cu" "B.Cu") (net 42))
 (segment (start 144.018 92.456) (end 144.018 105.156) (width 0.205232) (layer "B.Cu") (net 42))
 (segment (start 146.558 89.916) (end 144.018 92.456) (width 0.205232) (layer "B.Cu") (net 42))
 (segment (start 142.24 106.934) (end 141.986 106.934) (width 0.205232) (layer "B.Cu") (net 42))
 (segment (start 146.558 88.9) (end 146.558 89.916) (width 0.205232) (layer "B.Cu") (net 42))
 (segment (start 144.018 105.156) (end 142.24 106.934) (width 0.205232) (layer "B.Cu") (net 42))
 (via (at 144.585 90.25) (size 0.6) (drill 0.3) (layers "F.Cu" "B.Cu") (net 13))
 (segment (start 144.585 89.323) (end 145.008 88.9) (width 0.205232) (layer "B.Cu") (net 13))
 (segment (start 144.585 90.25) (end 144.585 89.323) (width 0.205232) (layer "B.Cu") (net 13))
 (segment (start 139.445 106.935) (end 139.446 106.934) (width 0.205232) (layer "F.Cu") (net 11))
 (segment (start 139.445 108.895) (end 139.445 106.935) (width 0.205232) (layer "F.Cu") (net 11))
 (via (at 141.855 90.25) (size 0.6) (drill 0.3) (layers "F.Cu" "B.Cu") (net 11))
 (via (at 139.446 106.934) (size 0.4) (drill 0.3) (layers "F.Cu" "B.Cu") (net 11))
 (segment (start 139.7 106.426) (end 140.462 106.426) (width 0.205232) (layer "B.Cu") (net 11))
 (segment (start 141.855 105.033) (end 141.855 90.25) (width 0.205232) (layer "B.Cu") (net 11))
 (segment (start 139.446 106.68) (end 139.7 106.426) (width 0.205232) (layer "B.Cu") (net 11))
 (segment (start 140.462 106.426) (end 141.855 105.033) (width 0.205232) (layer "B.Cu") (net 11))
 (segment (start 139.446 106.934) (end 139.446 106.68) (width 0.205232) (layer "B.Cu") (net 11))
 (segment (start 138.945 108.895) (end 138.945 107.055) (width 0.205232) (layer "F.Cu") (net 10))
 (segment (start 138.945 107.055) (end 139 107) (width 0.205232) (layer "F.Cu") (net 10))
 (via (at 140.945 90.25) (size 0.6) (drill 0.3) (layers "F.Cu" "B.Cu") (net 10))
 (via (at 138.938 106.934) (size 0.4) (drill 0.3) (layers "F.Cu" "B.Cu") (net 10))
 (segment (start 138.938 106.172) (end 138.938 106.934) (width 0.205232) (layer "B.Cu") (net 10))
 (segment (start 140.208 105.918) (end 139.192 105.918) (width 0.205232) (layer "B.Cu") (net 10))
 (segment (start 140.945 105.181) (end 140.208 105.918) (width 0.205232) (layer "B.Cu") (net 10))
 (segment (start 140.945 90.25) (end 140.945 105.181) (width 0.205232) (layer "B.Cu") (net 10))
 (segment (start 139.192 105.918) (end 138.938 106.172) (width 0.205232) (layer "B.Cu") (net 10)))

